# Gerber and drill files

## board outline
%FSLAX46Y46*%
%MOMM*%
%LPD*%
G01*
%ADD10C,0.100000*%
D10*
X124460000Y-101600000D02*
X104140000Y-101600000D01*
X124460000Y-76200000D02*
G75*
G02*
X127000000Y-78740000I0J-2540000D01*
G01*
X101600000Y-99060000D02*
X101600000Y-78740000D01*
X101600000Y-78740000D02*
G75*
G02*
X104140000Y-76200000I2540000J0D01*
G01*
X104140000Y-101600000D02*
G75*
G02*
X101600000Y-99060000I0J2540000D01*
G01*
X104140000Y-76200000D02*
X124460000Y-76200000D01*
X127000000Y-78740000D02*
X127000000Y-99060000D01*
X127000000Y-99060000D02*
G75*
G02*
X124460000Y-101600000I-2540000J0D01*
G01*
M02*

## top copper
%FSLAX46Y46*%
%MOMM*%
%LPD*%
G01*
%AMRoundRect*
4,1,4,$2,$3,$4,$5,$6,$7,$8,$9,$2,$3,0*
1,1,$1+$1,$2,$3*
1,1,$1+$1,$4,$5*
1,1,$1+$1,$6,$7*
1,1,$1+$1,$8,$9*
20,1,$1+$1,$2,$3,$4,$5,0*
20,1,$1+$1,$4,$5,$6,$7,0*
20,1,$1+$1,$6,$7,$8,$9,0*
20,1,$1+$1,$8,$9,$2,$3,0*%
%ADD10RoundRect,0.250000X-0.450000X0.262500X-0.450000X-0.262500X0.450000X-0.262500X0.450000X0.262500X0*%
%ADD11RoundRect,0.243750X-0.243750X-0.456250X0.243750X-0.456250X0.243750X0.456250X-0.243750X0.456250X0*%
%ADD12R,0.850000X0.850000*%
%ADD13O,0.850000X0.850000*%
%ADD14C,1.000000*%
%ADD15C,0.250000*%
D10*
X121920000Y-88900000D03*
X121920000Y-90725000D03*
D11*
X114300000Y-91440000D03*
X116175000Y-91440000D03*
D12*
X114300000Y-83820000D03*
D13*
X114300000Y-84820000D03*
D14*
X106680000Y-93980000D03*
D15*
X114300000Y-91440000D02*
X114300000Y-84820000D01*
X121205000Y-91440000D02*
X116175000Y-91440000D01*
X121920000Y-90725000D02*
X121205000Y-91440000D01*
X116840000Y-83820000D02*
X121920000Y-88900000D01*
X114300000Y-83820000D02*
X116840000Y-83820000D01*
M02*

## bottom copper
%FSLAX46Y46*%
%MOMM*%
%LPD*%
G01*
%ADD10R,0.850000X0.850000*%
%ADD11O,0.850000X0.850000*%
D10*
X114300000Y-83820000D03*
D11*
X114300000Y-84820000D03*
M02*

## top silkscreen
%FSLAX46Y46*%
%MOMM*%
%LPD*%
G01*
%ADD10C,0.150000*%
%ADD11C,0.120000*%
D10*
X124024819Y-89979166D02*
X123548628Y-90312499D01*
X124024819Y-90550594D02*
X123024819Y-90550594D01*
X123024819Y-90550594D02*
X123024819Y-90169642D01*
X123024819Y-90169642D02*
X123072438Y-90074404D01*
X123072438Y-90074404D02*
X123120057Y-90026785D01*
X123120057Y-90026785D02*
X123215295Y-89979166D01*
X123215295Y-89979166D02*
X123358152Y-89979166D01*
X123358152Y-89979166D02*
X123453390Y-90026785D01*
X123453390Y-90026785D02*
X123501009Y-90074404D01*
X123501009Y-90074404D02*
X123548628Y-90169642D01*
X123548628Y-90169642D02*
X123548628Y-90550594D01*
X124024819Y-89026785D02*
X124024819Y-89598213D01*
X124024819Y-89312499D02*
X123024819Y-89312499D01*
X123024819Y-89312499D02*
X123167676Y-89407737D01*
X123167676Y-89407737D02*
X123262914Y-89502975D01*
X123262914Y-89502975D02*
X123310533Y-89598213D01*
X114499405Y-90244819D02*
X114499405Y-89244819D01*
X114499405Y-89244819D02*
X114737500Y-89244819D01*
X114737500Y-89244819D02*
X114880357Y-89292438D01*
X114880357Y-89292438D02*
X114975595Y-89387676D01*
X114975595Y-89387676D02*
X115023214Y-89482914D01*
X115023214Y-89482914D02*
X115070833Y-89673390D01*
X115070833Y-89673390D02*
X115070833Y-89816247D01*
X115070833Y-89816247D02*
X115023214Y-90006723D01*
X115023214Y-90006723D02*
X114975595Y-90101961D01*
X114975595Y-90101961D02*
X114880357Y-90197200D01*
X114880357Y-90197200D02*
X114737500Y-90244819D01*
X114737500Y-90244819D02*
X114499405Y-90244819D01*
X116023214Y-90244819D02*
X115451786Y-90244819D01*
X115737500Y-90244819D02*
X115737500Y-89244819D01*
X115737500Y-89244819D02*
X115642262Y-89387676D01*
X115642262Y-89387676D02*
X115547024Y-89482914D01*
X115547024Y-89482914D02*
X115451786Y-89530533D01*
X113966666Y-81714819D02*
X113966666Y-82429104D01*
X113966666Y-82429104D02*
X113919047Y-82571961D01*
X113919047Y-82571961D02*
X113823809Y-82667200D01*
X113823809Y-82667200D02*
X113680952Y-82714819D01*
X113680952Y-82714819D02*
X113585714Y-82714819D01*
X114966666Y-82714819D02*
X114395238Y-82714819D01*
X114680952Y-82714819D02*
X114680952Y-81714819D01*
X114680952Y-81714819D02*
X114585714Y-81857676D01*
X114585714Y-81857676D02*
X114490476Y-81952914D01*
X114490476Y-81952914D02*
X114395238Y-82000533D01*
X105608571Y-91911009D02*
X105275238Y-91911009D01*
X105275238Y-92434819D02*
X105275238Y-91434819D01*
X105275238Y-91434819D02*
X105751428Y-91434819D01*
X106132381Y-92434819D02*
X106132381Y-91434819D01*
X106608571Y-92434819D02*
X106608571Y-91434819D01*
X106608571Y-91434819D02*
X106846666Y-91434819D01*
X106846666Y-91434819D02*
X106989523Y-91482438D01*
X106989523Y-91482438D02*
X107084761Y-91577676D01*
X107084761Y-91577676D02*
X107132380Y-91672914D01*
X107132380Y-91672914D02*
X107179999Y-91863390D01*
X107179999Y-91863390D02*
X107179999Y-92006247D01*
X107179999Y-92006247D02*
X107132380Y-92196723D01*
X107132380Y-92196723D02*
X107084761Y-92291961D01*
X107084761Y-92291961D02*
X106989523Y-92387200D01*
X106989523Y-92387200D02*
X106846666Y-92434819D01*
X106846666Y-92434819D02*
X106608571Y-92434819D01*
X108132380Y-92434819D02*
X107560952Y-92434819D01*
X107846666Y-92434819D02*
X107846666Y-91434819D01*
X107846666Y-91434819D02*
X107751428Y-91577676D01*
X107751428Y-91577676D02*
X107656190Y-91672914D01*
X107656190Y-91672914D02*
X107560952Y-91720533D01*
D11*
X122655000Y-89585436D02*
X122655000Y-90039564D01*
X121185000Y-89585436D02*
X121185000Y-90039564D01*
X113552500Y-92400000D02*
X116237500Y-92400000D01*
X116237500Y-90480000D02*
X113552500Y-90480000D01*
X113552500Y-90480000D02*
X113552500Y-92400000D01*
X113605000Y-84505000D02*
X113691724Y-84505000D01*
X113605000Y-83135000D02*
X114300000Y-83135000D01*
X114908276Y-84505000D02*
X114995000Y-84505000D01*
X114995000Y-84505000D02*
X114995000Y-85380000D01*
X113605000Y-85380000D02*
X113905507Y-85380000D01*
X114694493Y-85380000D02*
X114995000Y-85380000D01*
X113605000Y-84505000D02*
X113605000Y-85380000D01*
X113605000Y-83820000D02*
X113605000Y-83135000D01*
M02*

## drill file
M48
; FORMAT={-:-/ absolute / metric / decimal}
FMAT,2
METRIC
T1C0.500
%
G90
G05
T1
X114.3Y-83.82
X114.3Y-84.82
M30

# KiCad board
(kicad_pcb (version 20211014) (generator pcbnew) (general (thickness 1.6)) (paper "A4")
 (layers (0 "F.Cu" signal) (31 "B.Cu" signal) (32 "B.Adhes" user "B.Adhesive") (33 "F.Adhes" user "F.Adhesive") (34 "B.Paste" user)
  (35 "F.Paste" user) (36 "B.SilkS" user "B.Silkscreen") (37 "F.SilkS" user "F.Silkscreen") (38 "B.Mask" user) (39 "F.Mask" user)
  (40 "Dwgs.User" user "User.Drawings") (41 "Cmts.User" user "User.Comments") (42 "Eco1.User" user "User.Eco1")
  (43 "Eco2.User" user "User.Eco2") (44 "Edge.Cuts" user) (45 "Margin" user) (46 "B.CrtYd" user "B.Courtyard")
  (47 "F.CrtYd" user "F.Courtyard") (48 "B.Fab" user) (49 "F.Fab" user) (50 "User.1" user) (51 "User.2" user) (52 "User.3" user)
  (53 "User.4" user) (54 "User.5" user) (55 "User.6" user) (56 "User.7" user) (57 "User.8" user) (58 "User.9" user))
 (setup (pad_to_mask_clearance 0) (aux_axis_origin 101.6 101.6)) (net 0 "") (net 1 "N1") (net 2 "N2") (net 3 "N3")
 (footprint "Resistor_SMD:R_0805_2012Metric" (layer "F.Cu") (at 121.92 89.8125 -90)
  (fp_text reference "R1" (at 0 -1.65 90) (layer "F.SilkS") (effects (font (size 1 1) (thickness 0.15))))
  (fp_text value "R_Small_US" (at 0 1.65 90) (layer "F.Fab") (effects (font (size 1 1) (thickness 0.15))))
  (fp_line (start -0.227064 -0.735) (end 0.227064 -0.735) (layer "F.SilkS") (width 0.12))
  (fp_line (start -0.227064 0.735) (end 0.227064 0.735) (layer "F.SilkS") (width 0.12))
  (pad "1" smd roundrect (at -0.9125 0 270) (size 1.025 1.4) (layers "F.Cu" "F.Paste" "F.Mask") (roundrect_rratio 0.243902) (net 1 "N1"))
  (pad "2" smd roundrect (at 0.9125 0 270) (size 1.025 1.4) (layers "F.Cu" "F.Paste" "F.Mask") (roundrect_rratio 0.243902) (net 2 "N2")))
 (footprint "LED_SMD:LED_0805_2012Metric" (layer "F.Cu") (at 115.2375 91.44)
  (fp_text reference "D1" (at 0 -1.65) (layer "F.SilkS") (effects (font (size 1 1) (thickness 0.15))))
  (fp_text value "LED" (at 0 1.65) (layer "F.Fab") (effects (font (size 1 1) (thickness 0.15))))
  (fp_line (start -1.685 0.96) (end 1 0.96) (layer "F.SilkS") (width 0.12))
  (fp_line (start 1 -0.96) (end -1.685 -0.96) (layer "F.SilkS") (width 0.12))
  (fp_line (start -1.685 -0.96) (end -1.685 0.96) (layer "F.SilkS") (width 0.12))
  (pad "1" smd roundrect (at -0.9375 0) (size 0.975 1.4) (layers "F.Cu" "F.Paste" "F.Mask") (roundrect_rratio 0.25) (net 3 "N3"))
  (pad "2" smd roundrect (at 0.9375 0) (size 0.975 1.4) (layers "F.Cu" "F.Paste" "F.Mask") (roundrect_rratio 0.25) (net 2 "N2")))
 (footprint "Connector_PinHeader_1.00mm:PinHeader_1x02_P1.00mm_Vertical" (layer "F.Cu") (at 114.3 83.82)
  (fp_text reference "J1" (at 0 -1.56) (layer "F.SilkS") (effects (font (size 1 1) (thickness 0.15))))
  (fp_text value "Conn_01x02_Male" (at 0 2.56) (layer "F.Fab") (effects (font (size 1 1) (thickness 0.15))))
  (fp_line (start -0.695 0.685) (end -0.608276 0.685) (layer "F.SilkS") (width 0.12))
  (fp_line (start -0.695 -0.685) (end 0 -0.685) (layer "F.SilkS") (width 0.12))
  (fp_line (start 0.608276 0.685) (end 0.695 0.685) (layer "F.SilkS") (width 0.12))
  (fp_line (start 0.695 0.685) (end 0.695 1.56) (layer "F.SilkS") (width 0.12))
  (fp_line (start -0.695 1.56) (end -0.394493 1.56) (layer "F.SilkS") (width 0.12))
  (fp_line (start 0.394493 1.56) (end 0.695 1.56) (layer "F.SilkS") (width 0.12))
  (fp_line (start -0.695 0.685) (end -0.695 1.56) (layer "F.SilkS") (width 0.12))
  (fp_line (start -0.695 0) (end -0.695 -0.685) (layer "F.SilkS") (width 0.12))
  (pad "1" thru_hole rect (at 0 0) (size 0.85 0.85) (drill 0.5) (layers *.Cu *.Mask) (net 1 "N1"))
  (pad "2" thru_hole oval (at 0 1) (size 0.85 0.85) (drill 0.5) (layers *.Cu *.Mask) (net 3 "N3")))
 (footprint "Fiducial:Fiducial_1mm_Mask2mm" (layer "F.Cu") (at 106.68 93.98)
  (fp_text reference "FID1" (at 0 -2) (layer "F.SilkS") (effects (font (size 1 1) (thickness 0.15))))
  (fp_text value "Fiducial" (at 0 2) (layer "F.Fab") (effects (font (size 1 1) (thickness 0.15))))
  (pad "" smd circle (at 0 0) (size 1 1) (layers "F.Cu" "F.Mask") (solder_mask_margin 0.5) (clearance 0.5)))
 (gr_line (start 124.46 101.6) (end 104.14 101.6) (layer "Edge.Cuts") (width 0.1))
 (gr_arc (start 124.46 76.2) (mid 126.256051 76.943949) (end 127 78.74) (layer "Edge.Cuts") (width 0.1))
 (gr_line (start 101.6 99.06) (end 101.6 78.74) (layer "Edge.Cuts") (width 0.1))
 (gr_arc (start 101.6 78.74) (mid 102.343949 76.943949) (end 104.14 76.2) (layer "Edge.Cuts") (width 0.1))
 (gr_arc (start 104.14 101.6) (mid 102.343949 100.856051) (end 101.6 99.06) (layer "Edge.Cuts") (width 0.1))
 (gr_line (start 104.14 76.2) (end 124.46 76.2) (layer "Edge.Cuts") (width 0.1))
 (gr_line (start 127 78.74) (end 127 99.06) (layer "Edge.Cuts") (width 0.1))
 (gr_arc (start 127 99.06) (mid 126.256051 100.856051) (end 124.46 101.6) (layer "Edge.Cuts") (width 0.1))
 (segment (start 114.3 91.44) (end 114.3 84.82) (width 0.25) (layer "F.Cu") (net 3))
 (segment (start 121.205 91.44) (end 116.175 91.44) (width 0.25) (layer "F.Cu") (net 2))
 (segment (start 121.92 90.725) (end 121.205 91.44) (width 0.25) (layer "F.Cu") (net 2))
 (segment (start 116.84 83.82) (end 121.92 88.9) (width 0.25) (layer "F.Cu") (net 1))
 (segment (start 114.3 83.82) (end 116.84 83.82) (width 0.25) (layer "F.Cu") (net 1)))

